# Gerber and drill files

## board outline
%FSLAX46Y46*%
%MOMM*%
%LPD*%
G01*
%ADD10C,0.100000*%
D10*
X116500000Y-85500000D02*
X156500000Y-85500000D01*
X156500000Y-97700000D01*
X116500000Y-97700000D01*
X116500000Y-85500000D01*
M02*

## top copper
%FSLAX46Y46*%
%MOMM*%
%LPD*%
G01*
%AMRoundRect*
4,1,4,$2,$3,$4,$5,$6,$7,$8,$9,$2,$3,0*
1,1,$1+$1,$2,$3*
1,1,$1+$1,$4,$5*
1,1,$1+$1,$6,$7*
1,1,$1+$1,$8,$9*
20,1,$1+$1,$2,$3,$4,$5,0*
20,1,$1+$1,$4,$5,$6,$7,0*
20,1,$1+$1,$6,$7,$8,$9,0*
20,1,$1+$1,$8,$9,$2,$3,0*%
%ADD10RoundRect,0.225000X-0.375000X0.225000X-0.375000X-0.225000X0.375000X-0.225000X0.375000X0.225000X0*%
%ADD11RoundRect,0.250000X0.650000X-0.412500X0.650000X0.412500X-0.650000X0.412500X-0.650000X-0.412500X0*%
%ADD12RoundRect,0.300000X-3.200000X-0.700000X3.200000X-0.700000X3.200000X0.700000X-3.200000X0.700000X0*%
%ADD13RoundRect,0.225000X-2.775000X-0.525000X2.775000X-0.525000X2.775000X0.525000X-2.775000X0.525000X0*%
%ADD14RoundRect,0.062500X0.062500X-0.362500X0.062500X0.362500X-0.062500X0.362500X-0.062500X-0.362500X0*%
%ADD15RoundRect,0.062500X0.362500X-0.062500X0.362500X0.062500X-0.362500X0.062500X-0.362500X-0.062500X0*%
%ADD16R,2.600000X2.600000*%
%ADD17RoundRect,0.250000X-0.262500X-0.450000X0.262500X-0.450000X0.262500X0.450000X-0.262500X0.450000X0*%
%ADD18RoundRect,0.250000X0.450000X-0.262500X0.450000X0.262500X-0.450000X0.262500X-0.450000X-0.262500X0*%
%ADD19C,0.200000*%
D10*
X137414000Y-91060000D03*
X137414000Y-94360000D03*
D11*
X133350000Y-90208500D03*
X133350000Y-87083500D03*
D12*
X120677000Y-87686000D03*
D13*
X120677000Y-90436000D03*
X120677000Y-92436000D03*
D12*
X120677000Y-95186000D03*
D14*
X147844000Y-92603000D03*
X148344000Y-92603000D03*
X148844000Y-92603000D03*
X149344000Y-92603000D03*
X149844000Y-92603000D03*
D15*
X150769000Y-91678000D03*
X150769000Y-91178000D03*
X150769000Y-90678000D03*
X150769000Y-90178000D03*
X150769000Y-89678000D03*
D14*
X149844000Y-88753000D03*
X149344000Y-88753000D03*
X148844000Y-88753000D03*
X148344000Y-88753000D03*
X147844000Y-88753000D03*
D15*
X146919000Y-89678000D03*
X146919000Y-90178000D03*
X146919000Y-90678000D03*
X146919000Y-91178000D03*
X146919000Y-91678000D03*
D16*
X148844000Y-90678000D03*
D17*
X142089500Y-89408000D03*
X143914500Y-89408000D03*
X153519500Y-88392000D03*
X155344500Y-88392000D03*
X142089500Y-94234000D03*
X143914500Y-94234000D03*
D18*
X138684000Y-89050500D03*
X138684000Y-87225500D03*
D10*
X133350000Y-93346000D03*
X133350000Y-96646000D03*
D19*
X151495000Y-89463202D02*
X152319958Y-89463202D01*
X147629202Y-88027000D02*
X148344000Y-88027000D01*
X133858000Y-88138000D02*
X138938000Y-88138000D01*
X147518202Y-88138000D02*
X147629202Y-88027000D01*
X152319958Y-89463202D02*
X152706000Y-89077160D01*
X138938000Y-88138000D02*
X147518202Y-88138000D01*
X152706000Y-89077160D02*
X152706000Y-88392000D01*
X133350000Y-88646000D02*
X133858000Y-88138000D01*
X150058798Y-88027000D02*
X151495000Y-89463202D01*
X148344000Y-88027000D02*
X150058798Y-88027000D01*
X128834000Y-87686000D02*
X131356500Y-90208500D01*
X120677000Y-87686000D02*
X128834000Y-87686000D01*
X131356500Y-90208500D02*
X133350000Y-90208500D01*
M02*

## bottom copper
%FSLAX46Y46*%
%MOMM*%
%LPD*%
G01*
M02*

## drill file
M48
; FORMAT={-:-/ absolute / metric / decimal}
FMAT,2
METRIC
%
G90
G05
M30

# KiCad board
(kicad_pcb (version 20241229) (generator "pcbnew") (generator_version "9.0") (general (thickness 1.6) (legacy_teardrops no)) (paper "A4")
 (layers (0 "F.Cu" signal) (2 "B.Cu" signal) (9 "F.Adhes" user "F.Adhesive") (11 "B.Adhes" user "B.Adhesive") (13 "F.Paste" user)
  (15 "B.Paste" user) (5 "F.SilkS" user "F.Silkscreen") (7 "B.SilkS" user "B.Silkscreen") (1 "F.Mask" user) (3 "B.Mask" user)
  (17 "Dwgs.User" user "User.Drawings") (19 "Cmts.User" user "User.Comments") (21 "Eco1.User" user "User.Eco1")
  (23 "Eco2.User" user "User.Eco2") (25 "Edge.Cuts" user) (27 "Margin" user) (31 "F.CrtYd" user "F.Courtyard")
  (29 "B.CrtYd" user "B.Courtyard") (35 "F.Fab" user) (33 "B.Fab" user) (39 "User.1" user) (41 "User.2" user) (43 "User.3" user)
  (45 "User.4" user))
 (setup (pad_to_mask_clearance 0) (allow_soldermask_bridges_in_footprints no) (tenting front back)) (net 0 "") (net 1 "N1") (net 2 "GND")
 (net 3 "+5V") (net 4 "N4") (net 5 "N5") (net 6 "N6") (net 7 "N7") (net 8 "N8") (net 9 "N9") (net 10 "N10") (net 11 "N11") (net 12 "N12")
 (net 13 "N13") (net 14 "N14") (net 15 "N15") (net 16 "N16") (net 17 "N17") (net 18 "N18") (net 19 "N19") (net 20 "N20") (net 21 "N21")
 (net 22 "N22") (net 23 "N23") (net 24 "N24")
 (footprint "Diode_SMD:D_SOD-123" (layer "F.Cu") (at 137.414 92.71 -90)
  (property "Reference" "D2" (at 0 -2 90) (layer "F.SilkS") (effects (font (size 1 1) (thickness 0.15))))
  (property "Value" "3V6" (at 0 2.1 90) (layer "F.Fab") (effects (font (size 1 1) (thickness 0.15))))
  (pad "1" smd roundrect (at -1.65 0 270) (size 0.9 1.2) (layers "F.Cu" "F.Mask" "F.Paste") (roundrect_rratio 0.25) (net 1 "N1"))
  (pad "2" smd roundrect (at 1.65 0 270) (size 0.9 1.2) (layers "F.Cu" "F.Mask" "F.Paste") (roundrect_rratio 0.25) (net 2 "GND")))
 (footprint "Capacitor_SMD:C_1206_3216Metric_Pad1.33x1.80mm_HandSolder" (layer "F.Cu") (at 133.35 88.646 90)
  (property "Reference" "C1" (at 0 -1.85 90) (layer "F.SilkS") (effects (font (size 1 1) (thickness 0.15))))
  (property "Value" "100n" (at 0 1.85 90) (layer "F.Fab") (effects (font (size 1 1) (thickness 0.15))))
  (pad "1" smd roundrect (at -1.5625 0 90) (size 1.325 1.8) (layers "F.Cu" "F.Mask" "F.Paste") (roundrect_rratio 0.188679) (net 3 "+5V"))
  (pad "2" smd roundrect (at 1.5625 0 90) (size 1.325 1.8) (layers "F.Cu" "F.Mask" "F.Paste") (roundrect_rratio 0.188679) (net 2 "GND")))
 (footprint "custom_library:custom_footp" (layer "F.Cu") (at 120.677 91.436)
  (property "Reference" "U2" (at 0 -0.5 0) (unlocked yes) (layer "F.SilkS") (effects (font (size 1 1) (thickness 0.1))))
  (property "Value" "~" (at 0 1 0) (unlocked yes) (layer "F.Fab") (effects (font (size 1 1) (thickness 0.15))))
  (pad "1" smd roundrect (at 0 -3.75) (size 7 2) (layers "F.Cu" "F.Mask" "F.Paste") (roundrect_rratio 0.15) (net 3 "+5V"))
  (pad "2" smd roundrect (at 0 -1) (size 6 1.5) (layers "F.Cu" "F.Mask" "F.Paste") (roundrect_rratio 0.15) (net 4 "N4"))
  (pad "3" smd roundrect (at 0 1) (size 6 1.5) (layers "F.Cu" "F.Mask" "F.Paste") (roundrect_rratio 0.15) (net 1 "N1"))
  (pad "4" smd roundrect (at 0 3.75) (size 7 2) (layers "F.Cu" "F.Mask" "F.Paste") (roundrect_rratio 0.15) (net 2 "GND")))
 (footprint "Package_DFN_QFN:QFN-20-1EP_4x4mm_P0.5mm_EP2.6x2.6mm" (layer "F.Cu") (at 148.844 90.678 90)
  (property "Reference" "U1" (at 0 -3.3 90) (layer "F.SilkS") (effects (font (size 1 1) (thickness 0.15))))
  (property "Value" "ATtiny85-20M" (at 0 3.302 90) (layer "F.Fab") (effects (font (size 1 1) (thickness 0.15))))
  (pad "" smd roundrect (at -0.65 -0.65 90) (size 1.05 1.05) (layers "F.Paste") (roundrect_rratio 0.238095))
  (pad "" smd roundrect (at -0.65 0.65 90) (size 1.05 1.05) (layers "F.Paste") (roundrect_rratio 0.238095))
  (pad "" smd roundrect (at 0.65 -0.65 90) (size 1.05 1.05) (layers "F.Paste") (roundrect_rratio 0.238095))
  (pad "" smd roundrect (at 0.65 0.65 90) (size 1.05 1.05) (layers "F.Paste") (roundrect_rratio 0.238095))
  (pad "1" smd roundrect (at -1.925 -1 90) (size 0.85 0.25) (layers "F.Cu" "F.Mask" "F.Paste") (roundrect_rratio 0.25) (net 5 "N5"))
  (pad "2" smd roundrect (at -1.925 -0.5 90) (size 0.85 0.25) (layers "F.Cu" "F.Mask" "F.Paste") (roundrect_rratio 0.25) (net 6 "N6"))
  (pad "3" smd roundrect (at -1.925 0 90) (size 0.85 0.25) (layers "F.Cu" "F.Mask" "F.Paste") (roundrect_rratio 0.25) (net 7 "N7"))
  (pad "4" smd roundrect (at -1.925 0.5 90) (size 0.85 0.25) (layers "F.Cu" "F.Mask" "F.Paste") (roundrect_rratio 0.25) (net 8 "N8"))
  (pad "5" smd roundrect (at -1.925 1 90) (size 0.85 0.25) (layers "F.Cu" "F.Mask" "F.Paste") (roundrect_rratio 0.25) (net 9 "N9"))
  (pad "6" smd roundrect (at -1 1.925 90) (size 0.25 0.85) (layers "F.Cu" "F.Mask" "F.Paste") (roundrect_rratio 0.25) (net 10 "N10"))
  (pad "7" smd roundrect (at -0.5 1.925 90) (size 0.25 0.85) (layers "F.Cu" "F.Mask" "F.Paste") (roundrect_rratio 0.25) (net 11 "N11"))
  (pad "8" smd roundrect (at 0 1.925 90) (size 0.25 0.85) (layers "F.Cu" "F.Mask" "F.Paste") (roundrect_rratio 0.25) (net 2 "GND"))
  (pad "9" smd roundrect (at 0.5 1.925 90) (size 0.25 0.85) (layers "F.Cu" "F.Mask" "F.Paste") (roundrect_rratio 0.25) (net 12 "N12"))
  (pad "10" smd roundrect (at 1 1.925 90) (size 0.25 0.85) (layers "F.Cu" "F.Mask" "F.Paste") (roundrect_rratio 0.25) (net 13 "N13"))
  (pad "11" smd roundrect (at 1.925 1 90) (size 0.85 0.25) (layers "F.Cu" "F.Mask" "F.Paste") (roundrect_rratio 0.25) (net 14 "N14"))
  (pad "12" smd roundrect (at 1.925 0.5 90) (size 0.85 0.25) (layers "F.Cu" "F.Mask" "F.Paste") (roundrect_rratio 0.25) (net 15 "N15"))
  (pad "13" smd roundrect (at 1.925 0 90) (size 0.85 0.25) (layers "F.Cu" "F.Mask" "F.Paste") (roundrect_rratio 0.25) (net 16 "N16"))
  (pad "14" smd roundrect (at 1.925 -0.5 90) (size 0.85 0.25) (layers "F.Cu" "F.Mask" "F.Paste") (roundrect_rratio 0.25) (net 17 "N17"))
  (pad "15" smd roundrect (at 1.925 -1 90) (size 0.85 0.25) (layers "F.Cu" "F.Mask" "F.Paste") (roundrect_rratio 0.25) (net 3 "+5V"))
  (pad "16" smd roundrect (at 1 -1.925 90) (size 0.25 0.85) (layers "F.Cu" "F.Mask" "F.Paste") (roundrect_rratio 0.25) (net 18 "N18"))
  (pad "17" smd roundrect (at 0.5 -1.925 90) (size 0.25 0.85) (layers "F.Cu" "F.Mask" "F.Paste") (roundrect_rratio 0.25) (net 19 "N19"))
  (pad "18" smd roundrect (at 0 -1.925 90) (size 0.25 0.85) (layers "F.Cu" "F.Mask" "F.Paste") (roundrect_rratio 0.25) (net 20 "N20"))
  (pad "19" smd roundrect (at -0.5 -1.925 90) (size 0.25 0.85) (layers "F.Cu" "F.Mask" "F.Paste") (roundrect_rratio 0.25) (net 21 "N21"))
  (pad "20" smd roundrect (at -1 -1.925 90) (size 0.25 0.85) (layers "F.Cu" "F.Mask" "F.Paste") (roundrect_rratio 0.25) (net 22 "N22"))
  (pad "21" smd rect (at 0 0 90) (size 2.6 2.6) (layers "F.Cu" "F.Mask") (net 2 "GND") (zone_connect 2)))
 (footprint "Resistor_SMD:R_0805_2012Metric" (layer "F.Cu") (at 143.002 89.408)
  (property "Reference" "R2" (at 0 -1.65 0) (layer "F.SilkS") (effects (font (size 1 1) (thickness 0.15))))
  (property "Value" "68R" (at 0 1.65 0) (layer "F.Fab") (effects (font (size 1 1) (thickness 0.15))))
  (pad "1" smd roundrect (at -0.9125 0) (size 1.025 1.4) (layers "F.Cu" "F.Mask" "F.Paste") (roundrect_rratio 0.243902) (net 6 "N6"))
  (pad "2" smd roundrect (at 0.9125 0) (size 1.025 1.4) (layers "F.Cu" "F.Mask" "F.Paste") (roundrect_rratio 0.243902) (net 4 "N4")))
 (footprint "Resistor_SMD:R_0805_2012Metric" (layer "F.Cu") (at 154.432 88.392)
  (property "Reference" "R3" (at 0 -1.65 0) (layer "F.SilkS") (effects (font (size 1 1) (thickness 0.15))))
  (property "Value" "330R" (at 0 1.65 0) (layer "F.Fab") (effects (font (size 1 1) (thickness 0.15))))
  (pad "1" smd roundrect (at -0.9125 0) (size 1.025 1.4) (layers "F.Cu" "F.Mask" "F.Paste") (roundrect_rratio 0.243902) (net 15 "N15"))
  (pad "2" smd roundrect (at 0.9125 0) (size 1.025 1.4) (layers "F.Cu" "F.Mask" "F.Paste") (roundrect_rratio 0.243902) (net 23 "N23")))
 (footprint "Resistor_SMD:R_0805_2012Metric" (layer "F.Cu") (at 143.002 94.234)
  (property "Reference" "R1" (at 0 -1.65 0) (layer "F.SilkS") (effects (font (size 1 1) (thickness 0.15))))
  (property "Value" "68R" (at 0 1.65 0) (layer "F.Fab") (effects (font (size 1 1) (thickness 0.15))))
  (pad "1" smd roundrect (at -0.9125 0) (size 1.025 1.4) (layers "F.Cu" "F.Mask" "F.Paste") (roundrect_rratio 0.243902) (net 9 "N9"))
  (pad "2" smd roundrect (at 0.9125 0) (size 1.025 1.4) (layers "F.Cu" "F.Mask" "F.Paste") (roundrect_rratio 0.243902) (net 1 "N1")))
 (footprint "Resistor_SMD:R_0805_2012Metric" (layer "F.Cu") (at 138.684 88.138 90)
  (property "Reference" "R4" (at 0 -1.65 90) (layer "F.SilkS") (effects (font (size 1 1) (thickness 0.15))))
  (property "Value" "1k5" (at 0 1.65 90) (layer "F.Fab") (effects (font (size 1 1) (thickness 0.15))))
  (pad "1" smd roundrect (at -0.9125 0 90) (size 1.025 1.4) (layers "F.Cu" "F.Mask" "F.Paste") (roundrect_rratio 0.243902) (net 3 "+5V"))
  (pad "2" smd roundrect (at 0.9125 0 90) (size 1.025 1.4) (layers "F.Cu" "F.Mask" "F.Paste") (roundrect_rratio 0.243902) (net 4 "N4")))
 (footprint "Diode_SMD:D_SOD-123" (layer "F.Cu") (at 133.35 94.996 -90)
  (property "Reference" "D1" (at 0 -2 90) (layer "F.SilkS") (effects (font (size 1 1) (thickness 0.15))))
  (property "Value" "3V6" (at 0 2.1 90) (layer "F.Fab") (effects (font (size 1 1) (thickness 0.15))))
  (pad "1" smd roundrect (at -1.65 0 270) (size 0.9 1.2) (layers "F.Cu" "F.Mask" "F.Paste") (roundrect_rratio 0.25) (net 4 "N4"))
  (pad "2" smd roundrect (at 1.65 0 270) (size 0.9 1.2) (layers "F.Cu" "F.Mask" "F.Paste") (roundrect_rratio 0.25) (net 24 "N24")))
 (gr_rect (start 116.5 85.5) (end 156.5 97.7) (stroke (width 0.1) (type solid)) (fill no) (layer "Edge.Cuts"))
 (segment (start 151.495 89.463202) (end 152.319958 89.463202) (width 0.2) (layer "F.Cu") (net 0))
 (segment (start 147.629202 88.027) (end 148.344 88.027) (width 0.2) (layer "F.Cu") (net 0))
 (segment (start 133.858 88.138) (end 138.938 88.138) (width 0.2) (layer "F.Cu") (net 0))
 (segment (start 147.518202 88.138) (end 147.629202 88.027) (width 0.2) (layer "F.Cu") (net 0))
 (segment (start 152.319958 89.463202) (end 152.706 89.07716) (width 0.2) (layer "F.Cu") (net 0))
 (segment (start 138.938 88.138) (end 147.518202 88.138) (width 0.2) (layer "F.Cu") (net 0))
 (segment (start 152.706 89.07716) (end 152.706 88.392) (width 0.2) (layer "F.Cu") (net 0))
 (segment (start 133.35 88.646) (end 133.858 88.138) (width 0.2) (layer "F.Cu") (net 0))
 (segment (start 150.058798 88.027) (end 151.495 89.463202) (width 0.2) (layer "F.Cu") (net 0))
 (segment (start 148.344 88.027) (end 150.058798 88.027) (width 0.2) (layer "F.Cu") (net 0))
 (segment (start 128.834 87.686) (end 131.3565 90.2085) (width 0.2) (layer "F.Cu") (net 3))
 (segment (start 120.677 87.686) (end 128.834 87.686) (width 0.2) (layer "F.Cu") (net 3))
 (segment (start 131.3565 90.2085) (end 133.35 90.2085) (width 0.2) (layer "F.Cu") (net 3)))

